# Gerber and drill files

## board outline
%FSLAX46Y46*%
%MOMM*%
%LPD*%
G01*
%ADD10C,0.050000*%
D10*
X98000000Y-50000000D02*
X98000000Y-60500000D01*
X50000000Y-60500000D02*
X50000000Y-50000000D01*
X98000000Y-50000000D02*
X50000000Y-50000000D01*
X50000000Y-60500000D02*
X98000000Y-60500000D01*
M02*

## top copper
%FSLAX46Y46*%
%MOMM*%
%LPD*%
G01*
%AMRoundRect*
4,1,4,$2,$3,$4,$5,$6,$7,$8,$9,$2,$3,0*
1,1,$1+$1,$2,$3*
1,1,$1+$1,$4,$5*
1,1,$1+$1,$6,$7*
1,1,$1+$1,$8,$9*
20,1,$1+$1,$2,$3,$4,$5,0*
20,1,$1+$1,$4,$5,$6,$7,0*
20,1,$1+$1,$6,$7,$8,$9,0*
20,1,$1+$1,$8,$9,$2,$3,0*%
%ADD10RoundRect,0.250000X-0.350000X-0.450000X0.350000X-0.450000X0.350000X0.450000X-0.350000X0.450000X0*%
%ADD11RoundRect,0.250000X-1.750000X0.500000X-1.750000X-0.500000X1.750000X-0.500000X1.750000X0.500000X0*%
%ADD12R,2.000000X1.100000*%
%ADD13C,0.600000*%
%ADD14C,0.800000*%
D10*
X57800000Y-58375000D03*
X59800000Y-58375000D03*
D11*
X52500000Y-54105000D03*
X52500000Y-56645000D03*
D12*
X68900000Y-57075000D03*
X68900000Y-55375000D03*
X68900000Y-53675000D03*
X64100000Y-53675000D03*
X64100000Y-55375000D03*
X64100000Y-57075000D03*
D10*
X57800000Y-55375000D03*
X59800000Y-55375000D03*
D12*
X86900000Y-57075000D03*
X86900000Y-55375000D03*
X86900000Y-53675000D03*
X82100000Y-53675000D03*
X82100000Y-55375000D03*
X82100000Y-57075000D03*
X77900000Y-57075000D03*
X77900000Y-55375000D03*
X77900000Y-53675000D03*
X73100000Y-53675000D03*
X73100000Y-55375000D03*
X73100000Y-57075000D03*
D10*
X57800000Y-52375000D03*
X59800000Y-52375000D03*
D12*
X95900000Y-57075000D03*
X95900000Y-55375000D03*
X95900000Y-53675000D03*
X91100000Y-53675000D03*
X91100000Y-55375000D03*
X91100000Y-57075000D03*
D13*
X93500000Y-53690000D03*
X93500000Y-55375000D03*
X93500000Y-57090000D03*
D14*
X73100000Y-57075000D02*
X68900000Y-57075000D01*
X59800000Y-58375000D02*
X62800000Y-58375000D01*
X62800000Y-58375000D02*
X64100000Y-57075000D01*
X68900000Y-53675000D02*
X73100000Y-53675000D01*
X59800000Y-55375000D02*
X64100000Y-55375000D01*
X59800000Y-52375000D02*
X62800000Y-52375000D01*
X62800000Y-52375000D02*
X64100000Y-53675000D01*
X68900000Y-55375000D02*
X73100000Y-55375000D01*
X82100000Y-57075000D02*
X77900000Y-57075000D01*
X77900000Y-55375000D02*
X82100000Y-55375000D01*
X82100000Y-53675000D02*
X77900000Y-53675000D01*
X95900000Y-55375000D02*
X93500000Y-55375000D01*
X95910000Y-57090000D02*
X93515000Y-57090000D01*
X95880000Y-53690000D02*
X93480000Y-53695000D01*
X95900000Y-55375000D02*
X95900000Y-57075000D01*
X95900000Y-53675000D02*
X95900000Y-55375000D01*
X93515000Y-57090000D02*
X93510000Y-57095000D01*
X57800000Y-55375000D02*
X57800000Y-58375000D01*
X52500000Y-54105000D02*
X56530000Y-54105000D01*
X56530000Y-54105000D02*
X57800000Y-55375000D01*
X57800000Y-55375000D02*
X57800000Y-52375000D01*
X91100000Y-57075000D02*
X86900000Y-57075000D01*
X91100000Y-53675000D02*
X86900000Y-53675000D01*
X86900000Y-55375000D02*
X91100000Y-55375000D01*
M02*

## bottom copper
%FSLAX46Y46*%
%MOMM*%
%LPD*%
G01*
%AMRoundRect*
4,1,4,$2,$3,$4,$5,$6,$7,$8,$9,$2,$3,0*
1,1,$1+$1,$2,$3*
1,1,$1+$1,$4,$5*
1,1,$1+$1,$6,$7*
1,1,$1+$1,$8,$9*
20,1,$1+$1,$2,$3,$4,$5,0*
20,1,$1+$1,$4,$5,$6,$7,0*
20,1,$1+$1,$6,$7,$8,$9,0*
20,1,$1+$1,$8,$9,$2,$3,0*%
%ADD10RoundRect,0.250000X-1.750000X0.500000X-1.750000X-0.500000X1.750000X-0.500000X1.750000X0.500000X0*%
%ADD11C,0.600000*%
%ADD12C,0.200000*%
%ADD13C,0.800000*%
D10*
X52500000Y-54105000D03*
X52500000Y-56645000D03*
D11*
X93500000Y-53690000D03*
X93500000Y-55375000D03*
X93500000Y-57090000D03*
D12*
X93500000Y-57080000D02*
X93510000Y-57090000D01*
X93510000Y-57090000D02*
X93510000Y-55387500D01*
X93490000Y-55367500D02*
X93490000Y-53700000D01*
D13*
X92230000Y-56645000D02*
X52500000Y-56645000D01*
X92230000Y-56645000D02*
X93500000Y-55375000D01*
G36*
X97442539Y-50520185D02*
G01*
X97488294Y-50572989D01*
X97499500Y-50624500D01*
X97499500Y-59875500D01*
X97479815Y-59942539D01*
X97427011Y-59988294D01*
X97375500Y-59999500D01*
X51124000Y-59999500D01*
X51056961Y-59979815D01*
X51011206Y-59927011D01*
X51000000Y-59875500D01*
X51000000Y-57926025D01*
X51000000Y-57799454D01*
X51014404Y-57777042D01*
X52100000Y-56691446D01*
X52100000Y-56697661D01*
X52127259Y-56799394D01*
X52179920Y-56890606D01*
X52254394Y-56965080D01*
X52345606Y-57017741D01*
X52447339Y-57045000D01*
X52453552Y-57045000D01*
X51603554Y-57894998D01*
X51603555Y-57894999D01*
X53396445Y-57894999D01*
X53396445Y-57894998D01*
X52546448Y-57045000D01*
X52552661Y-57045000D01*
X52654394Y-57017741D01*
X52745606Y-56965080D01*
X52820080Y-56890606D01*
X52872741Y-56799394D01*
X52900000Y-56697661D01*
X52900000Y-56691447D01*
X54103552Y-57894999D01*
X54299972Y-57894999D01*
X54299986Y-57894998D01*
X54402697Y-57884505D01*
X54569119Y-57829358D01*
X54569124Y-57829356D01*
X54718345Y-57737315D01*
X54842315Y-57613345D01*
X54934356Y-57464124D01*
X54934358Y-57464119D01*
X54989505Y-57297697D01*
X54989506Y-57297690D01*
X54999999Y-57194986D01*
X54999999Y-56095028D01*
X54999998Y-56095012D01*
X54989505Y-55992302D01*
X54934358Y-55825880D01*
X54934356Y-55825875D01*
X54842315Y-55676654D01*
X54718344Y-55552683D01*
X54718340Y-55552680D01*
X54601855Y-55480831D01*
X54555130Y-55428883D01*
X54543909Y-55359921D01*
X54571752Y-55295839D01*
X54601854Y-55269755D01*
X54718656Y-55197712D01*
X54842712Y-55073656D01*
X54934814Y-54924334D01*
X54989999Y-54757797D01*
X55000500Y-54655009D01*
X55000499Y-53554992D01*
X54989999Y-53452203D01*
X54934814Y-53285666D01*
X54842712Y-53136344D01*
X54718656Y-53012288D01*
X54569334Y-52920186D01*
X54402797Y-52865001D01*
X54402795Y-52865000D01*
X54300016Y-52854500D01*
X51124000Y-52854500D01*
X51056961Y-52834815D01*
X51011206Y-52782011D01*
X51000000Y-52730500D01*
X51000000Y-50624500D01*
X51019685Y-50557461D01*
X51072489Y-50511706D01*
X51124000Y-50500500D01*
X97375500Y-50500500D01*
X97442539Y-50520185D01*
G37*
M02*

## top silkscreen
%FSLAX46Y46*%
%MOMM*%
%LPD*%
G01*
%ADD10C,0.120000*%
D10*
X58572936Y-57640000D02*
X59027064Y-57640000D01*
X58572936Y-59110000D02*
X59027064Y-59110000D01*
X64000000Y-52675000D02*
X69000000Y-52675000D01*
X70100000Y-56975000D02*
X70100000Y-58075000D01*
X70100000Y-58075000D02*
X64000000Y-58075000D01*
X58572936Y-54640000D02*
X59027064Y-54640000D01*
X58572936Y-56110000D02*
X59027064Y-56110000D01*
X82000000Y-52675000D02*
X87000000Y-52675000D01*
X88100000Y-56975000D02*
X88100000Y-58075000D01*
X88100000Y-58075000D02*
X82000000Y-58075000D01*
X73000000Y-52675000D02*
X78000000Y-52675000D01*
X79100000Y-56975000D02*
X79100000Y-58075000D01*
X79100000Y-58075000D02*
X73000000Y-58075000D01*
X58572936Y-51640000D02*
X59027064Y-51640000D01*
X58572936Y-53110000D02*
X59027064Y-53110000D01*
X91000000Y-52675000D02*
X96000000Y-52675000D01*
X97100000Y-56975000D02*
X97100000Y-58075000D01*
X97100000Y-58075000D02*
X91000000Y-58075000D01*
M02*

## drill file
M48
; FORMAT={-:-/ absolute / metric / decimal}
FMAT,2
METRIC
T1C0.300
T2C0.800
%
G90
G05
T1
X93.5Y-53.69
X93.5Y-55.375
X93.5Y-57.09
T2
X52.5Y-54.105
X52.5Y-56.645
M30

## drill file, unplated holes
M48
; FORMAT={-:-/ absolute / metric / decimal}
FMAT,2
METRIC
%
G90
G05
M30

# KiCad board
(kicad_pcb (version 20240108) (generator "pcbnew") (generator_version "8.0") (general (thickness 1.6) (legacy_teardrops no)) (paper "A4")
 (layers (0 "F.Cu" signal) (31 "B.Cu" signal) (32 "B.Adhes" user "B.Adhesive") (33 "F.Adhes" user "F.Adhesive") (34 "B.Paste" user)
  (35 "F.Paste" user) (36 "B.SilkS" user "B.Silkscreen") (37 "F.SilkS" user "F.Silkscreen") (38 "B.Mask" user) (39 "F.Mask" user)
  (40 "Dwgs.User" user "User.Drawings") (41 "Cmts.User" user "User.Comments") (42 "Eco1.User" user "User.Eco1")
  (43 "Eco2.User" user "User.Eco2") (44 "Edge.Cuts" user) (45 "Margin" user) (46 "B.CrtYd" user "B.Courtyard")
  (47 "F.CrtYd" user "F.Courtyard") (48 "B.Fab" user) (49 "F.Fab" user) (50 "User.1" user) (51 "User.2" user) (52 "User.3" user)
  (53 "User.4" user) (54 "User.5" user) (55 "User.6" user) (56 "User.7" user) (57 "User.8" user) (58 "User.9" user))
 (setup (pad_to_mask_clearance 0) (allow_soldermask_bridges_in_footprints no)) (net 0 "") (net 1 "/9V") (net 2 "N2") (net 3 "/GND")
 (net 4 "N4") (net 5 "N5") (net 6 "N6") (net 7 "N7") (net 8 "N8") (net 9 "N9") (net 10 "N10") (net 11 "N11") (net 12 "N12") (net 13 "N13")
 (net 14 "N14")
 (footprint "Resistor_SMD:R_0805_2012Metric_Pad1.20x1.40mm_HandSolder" (layer "F.Cu") (at 58.8 58.375)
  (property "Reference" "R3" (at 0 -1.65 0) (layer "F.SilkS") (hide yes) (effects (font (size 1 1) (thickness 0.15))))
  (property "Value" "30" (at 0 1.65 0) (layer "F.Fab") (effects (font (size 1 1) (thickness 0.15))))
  (fp_line (start -0.227064 -0.735) (end 0.227064 -0.735) (stroke (width 0.12) (type solid)) (layer "F.SilkS"))
  (fp_line (start -0.227064 0.735) (end 0.227064 0.735) (stroke (width 0.12) (type solid)) (layer "F.SilkS"))
  (pad "1" smd roundrect (at -1 0) (size 1.2 1.4) (layers "F.Cu" "F.Paste" "F.Mask") (roundrect_rratio 0.208333) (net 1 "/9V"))
  (pad "2" smd roundrect (at 1 0) (size 1.2 1.4) (layers "F.Cu" "F.Paste" "F.Mask") (roundrect_rratio 0.208333) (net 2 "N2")))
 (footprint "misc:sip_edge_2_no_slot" (layer "F.Cu") (at 50.5 55.375 -90)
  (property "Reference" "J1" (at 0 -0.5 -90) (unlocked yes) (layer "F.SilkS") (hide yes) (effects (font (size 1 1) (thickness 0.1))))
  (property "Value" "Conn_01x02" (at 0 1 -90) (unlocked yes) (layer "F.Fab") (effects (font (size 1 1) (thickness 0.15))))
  (pad "1" thru_hole roundrect (at -1.27 -2 270) (size 1.5 4) (drill 0.8) (layers "*.Cu" "*.Mask") (remove_unused_layers no)
   (roundrect_rratio 0.1666666667) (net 1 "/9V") (thermal_bridge_angle 45))
  (pad "2" thru_hole roundrect (at 1.27 -2 270) (size 1.5 4) (drill 0.8) (layers "*.Cu" "*.Mask") (remove_unused_layers no)
   (roundrect_rratio 0.1666666667) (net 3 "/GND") (thermal_bridge_angle 45)))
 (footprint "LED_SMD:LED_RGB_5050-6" (layer "F.Cu") (at 66.5 55.375 180)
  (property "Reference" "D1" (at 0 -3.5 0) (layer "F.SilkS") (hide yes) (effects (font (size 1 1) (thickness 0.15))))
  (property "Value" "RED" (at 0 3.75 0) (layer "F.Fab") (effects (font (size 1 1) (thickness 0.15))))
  (fp_line (start 2.5 2.7) (end -2.5 2.7) (stroke (width 0.12) (type solid)) (layer "F.SilkS"))
  (fp_line (start -3.6 -1.6) (end -3.6 -2.7) (stroke (width 0.12) (type solid)) (layer "F.SilkS"))
  (fp_line (start -3.6 -2.7) (end 2.5 -2.7) (stroke (width 0.12) (type solid)) (layer "F.SilkS"))
  (pad "1" smd rect (at -2.4 -1.7 270) (size 1.1 2) (layers "F.Cu" "F.Paste" "F.Mask") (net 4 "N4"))
  (pad "2" smd rect (at -2.4 0 270) (size 1.1 2) (layers "F.Cu" "F.Paste" "F.Mask") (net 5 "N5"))
  (pad "3" smd rect (at -2.4 1.7 270) (size 1.1 2) (layers "F.Cu" "F.Paste" "F.Mask") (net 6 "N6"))
  (pad "4" smd rect (at 2.4 1.7 270) (size 1.1 2) (layers "F.Cu" "F.Paste" "F.Mask") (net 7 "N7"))
  (pad "5" smd rect (at 2.4 0 270) (size 1.1 2) (layers "F.Cu" "F.Paste" "F.Mask") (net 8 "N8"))
  (pad "6" smd rect (at 2.4 -1.7 270) (size 1.1 2) (layers "F.Cu" "F.Paste" "F.Mask") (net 2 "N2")))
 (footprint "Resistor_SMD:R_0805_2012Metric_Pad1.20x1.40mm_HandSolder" (layer "F.Cu") (at 58.8 55.375)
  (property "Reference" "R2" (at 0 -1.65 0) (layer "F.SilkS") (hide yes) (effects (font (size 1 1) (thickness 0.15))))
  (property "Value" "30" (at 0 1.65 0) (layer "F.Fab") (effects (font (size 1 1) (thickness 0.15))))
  (fp_line (start -0.227064 -0.735) (end 0.227064 -0.735) (stroke (width 0.12) (type solid)) (layer "F.SilkS"))
  (fp_line (start -0.227064 0.735) (end 0.227064 0.735) (stroke (width 0.12) (type solid)) (layer "F.SilkS"))
  (pad "1" smd roundrect (at -1 0) (size 1.2 1.4) (layers "F.Cu" "F.Paste" "F.Mask") (roundrect_rratio 0.208333) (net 1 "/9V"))
  (pad "2" smd roundrect (at 1 0) (size 1.2 1.4) (layers "F.Cu" "F.Paste" "F.Mask") (roundrect_rratio 0.208333) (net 8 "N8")))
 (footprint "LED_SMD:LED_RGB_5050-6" (layer "F.Cu") (at 84.5 55.375 180)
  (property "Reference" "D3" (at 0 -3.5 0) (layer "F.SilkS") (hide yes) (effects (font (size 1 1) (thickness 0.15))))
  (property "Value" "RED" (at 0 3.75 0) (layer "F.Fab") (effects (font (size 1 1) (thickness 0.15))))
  (fp_line (start 2.5 2.7) (end -2.5 2.7) (stroke (width 0.12) (type solid)) (layer "F.SilkS"))
  (fp_line (start -3.6 -1.6) (end -3.6 -2.7) (stroke (width 0.12) (type solid)) (layer "F.SilkS"))
  (fp_line (start -3.6 -2.7) (end 2.5 -2.7) (stroke (width 0.12) (type solid)) (layer "F.SilkS"))
  (pad "1" smd rect (at -2.4 -1.7 270) (size 1.1 2) (layers "F.Cu" "F.Paste" "F.Mask") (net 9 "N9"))
  (pad "2" smd rect (at -2.4 0 270) (size 1.1 2) (layers "F.Cu" "F.Paste" "F.Mask") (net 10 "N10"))
  (pad "3" smd rect (at -2.4 1.7 270) (size 1.1 2) (layers "F.Cu" "F.Paste" "F.Mask") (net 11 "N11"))
  (pad "4" smd rect (at 2.4 1.7 270) (size 1.1 2) (layers "F.Cu" "F.Paste" "F.Mask") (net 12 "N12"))
  (pad "5" smd rect (at 2.4 0 270) (size 1.1 2) (layers "F.Cu" "F.Paste" "F.Mask") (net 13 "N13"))
  (pad "6" smd rect (at 2.4 -1.7 270) (size 1.1 2) (layers "F.Cu" "F.Paste" "F.Mask") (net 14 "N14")))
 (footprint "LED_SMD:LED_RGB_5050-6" (layer "F.Cu") (at 75.5 55.375 180)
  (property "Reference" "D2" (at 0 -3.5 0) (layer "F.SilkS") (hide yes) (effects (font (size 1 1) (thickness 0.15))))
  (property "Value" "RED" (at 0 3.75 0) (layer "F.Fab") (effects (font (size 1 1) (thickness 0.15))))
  (fp_line (start 2.5 2.7) (end -2.5 2.7) (stroke (width 0.12) (type solid)) (layer "F.SilkS"))
  (fp_line (start -3.6 -1.6) (end -3.6 -2.7) (stroke (width 0.12) (type solid)) (layer "F.SilkS"))
  (fp_line (start -3.6 -2.7) (end 2.5 -2.7) (stroke (width 0.12) (type solid)) (layer "F.SilkS"))
  (pad "1" smd rect (at -2.4 -1.7 270) (size 1.1 2) (layers "F.Cu" "F.Paste" "F.Mask") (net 14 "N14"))
  (pad "2" smd rect (at -2.4 0 270) (size 1.1 2) (layers "F.Cu" "F.Paste" "F.Mask") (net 13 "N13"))
  (pad "3" smd rect (at -2.4 1.7 270) (size 1.1 2) (layers "F.Cu" "F.Paste" "F.Mask") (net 12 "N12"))
  (pad "4" smd rect (at 2.4 1.7 270) (size 1.1 2) (layers "F.Cu" "F.Paste" "F.Mask") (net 6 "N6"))
  (pad "5" smd rect (at 2.4 0 270) (size 1.1 2) (layers "F.Cu" "F.Paste" "F.Mask") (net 5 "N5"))
  (pad "6" smd rect (at 2.4 -1.7 270) (size 1.1 2) (layers "F.Cu" "F.Paste" "F.Mask") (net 4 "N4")))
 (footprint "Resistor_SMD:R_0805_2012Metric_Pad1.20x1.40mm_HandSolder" (layer "F.Cu") (at 58.8 52.375)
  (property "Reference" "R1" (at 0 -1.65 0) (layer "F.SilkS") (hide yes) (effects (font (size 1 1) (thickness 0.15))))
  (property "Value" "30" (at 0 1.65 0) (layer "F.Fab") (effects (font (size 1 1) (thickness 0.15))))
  (fp_line (start -0.227064 -0.735) (end 0.227064 -0.735) (stroke (width 0.12) (type solid)) (layer "F.SilkS"))
  (fp_line (start -0.227064 0.735) (end 0.227064 0.735) (stroke (width 0.12) (type solid)) (layer "F.SilkS"))
  (pad "1" smd roundrect (at -1 0) (size 1.2 1.4) (layers "F.Cu" "F.Paste" "F.Mask") (roundrect_rratio 0.208333) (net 1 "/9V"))
  (pad "2" smd roundrect (at 1 0) (size 1.2 1.4) (layers "F.Cu" "F.Paste" "F.Mask") (roundrect_rratio 0.208333) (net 7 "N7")))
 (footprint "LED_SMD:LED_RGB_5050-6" (layer "F.Cu") (at 93.5 55.375 180)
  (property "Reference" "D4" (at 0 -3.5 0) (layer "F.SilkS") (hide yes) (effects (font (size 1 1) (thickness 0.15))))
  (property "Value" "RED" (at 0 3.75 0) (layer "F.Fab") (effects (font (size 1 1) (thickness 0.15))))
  (fp_line (start 2.5 2.7) (end -2.5 2.7) (stroke (width 0.12) (type solid)) (layer "F.SilkS"))
  (fp_line (start -3.6 -1.6) (end -3.6 -2.7) (stroke (width 0.12) (type solid)) (layer "F.SilkS"))
  (fp_line (start -3.6 -2.7) (end 2.5 -2.7) (stroke (width 0.12) (type solid)) (layer "F.SilkS"))
  (pad "1" smd rect (at -2.4 -1.7 270) (size 1.1 2) (layers "F.Cu" "F.Paste" "F.Mask") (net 3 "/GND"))
  (pad "2" smd rect (at -2.4 0 270) (size 1.1 2) (layers "F.Cu" "F.Paste" "F.Mask") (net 3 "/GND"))
  (pad "3" smd rect (at -2.4 1.7 270) (size 1.1 2) (layers "F.Cu" "F.Paste" "F.Mask") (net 3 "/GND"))
  (pad "4" smd rect (at 2.4 1.7 270) (size 1.1 2) (layers "F.Cu" "F.Paste" "F.Mask") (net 11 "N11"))
  (pad "5" smd rect (at 2.4 0 270) (size 1.1 2) (layers "F.Cu" "F.Paste" "F.Mask") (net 10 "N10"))
  (pad "6" smd rect (at 2.4 -1.7 270) (size 1.1 2) (layers "F.Cu" "F.Paste" "F.Mask") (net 9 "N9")))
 (gr_line (start 98 50) (end 98 60.5) (stroke (width 0.05) (type default)) (layer "Edge.Cuts"))
 (gr_line (start 50 60.5) (end 50 50) (stroke (width 0.05) (type default)) (layer "Edge.Cuts"))
 (gr_line (start 98 50) (end 50 50) (stroke (width 0.05) (type default)) (layer "Edge.Cuts"))
 (gr_line (start 50 60.5) (end 98 60.5) (stroke (width 0.05) (type default)) (layer "Edge.Cuts"))
 (segment (start 73.1 57.075) (end 68.9 57.075) (width 0.8) (layer "F.Cu") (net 4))
 (segment (start 59.8 58.375) (end 62.8 58.375) (width 0.8) (layer "F.Cu") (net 2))
 (segment (start 62.8 58.375) (end 64.1 57.075) (width 0.8) (layer "F.Cu") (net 2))
 (segment (start 68.9 53.675) (end 73.1 53.675) (width 0.8) (layer "F.Cu") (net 6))
 (segment (start 59.8 55.375) (end 64.1 55.375) (width 0.8) (layer "F.Cu") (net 8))
 (segment (start 59.8 52.375) (end 62.8 52.375) (width 0.8) (layer "F.Cu") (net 7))
 (segment (start 62.8 52.375) (end 64.1 53.675) (width 0.8) (layer "F.Cu") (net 7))
 (segment (start 68.9 55.375) (end 73.1 55.375) (width 0.8) (layer "F.Cu") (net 5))
 (segment (start 82.1 57.075) (end 77.9 57.075) (width 0.8) (layer "F.Cu") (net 14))
 (segment (start 77.9 55.375) (end 82.1 55.375) (width 0.8) (layer "F.Cu") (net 13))
 (segment (start 82.1 53.675) (end 77.9 53.675) (width 0.8) (layer "F.Cu") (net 12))
 (segment (start 95.9 55.375) (end 93.5 55.375) (width 0.8) (layer "F.Cu") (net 3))
 (segment (start 95.91 57.09) (end 93.515 57.09) (width 0.8) (layer "F.Cu") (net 3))
 (segment (start 95.88 53.69) (end 93.48 53.695) (width 0.8) (layer "F.Cu") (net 3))
 (segment (start 95.9 55.375) (end 95.9 57.075) (width 0.8) (layer "F.Cu") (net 3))
 (segment (start 95.9 53.675) (end 95.9 55.375) (width 0.8) (layer "F.Cu") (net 3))
 (segment (start 93.515 57.09) (end 93.51 57.095) (width 0.8) (layer "F.Cu") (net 3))
 (via (at 93.5 53.69) (size 0.6) (drill 0.3) (layers "F.Cu" "B.Cu") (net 3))
 (via (at 93.5 55.375) (size 0.6) (drill 0.3) (layers "F.Cu" "B.Cu") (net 3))
 (via (at 93.5 57.09) (size 0.6) (drill 0.3) (layers "F.Cu" "B.Cu") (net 3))
 (segment (start 93.5 57.08) (end 93.51 57.09) (width 0.2) (layer "B.Cu") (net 3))
 (segment (start 93.51 57.09) (end 93.51 55.3875) (width 0.2) (layer "B.Cu") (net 3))
 (segment (start 93.49 55.3675) (end 93.49 53.7) (width 0.2) (layer "B.Cu") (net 3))
 (segment (start 92.23 56.645) (end 52.5 56.645) (width 0.8) (layer "B.Cu") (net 3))
 (segment (start 92.23 56.645) (end 93.5 55.375) (width 0.8) (layer "B.Cu") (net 3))
 (segment (start 57.8 55.375) (end 57.8 58.375) (width 0.8) (layer "F.Cu") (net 1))
 (segment (start 52.5 54.105) (end 56.53 54.105) (width 0.8) (layer "F.Cu") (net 1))
 (segment (start 56.53 54.105) (end 57.8 55.375) (width 0.8) (layer "F.Cu") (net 1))
 (segment (start 57.8 55.375) (end 57.8 52.375) (width 0.8) (layer "F.Cu") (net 1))
 (segment (start 91.1 57.075) (end 86.9 57.075) (width 0.8) (layer "F.Cu") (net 9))
 (segment (start 91.1 53.675) (end 86.9 53.675) (width 0.8) (layer "F.Cu") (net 11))
 (segment (start 86.9 55.375) (end 91.1 55.375) (width 0.8) (layer "F.Cu") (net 10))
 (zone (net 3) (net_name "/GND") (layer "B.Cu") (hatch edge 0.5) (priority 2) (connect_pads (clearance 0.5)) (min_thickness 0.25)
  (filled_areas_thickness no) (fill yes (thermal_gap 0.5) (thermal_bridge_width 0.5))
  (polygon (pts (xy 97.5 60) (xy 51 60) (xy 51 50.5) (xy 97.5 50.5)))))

